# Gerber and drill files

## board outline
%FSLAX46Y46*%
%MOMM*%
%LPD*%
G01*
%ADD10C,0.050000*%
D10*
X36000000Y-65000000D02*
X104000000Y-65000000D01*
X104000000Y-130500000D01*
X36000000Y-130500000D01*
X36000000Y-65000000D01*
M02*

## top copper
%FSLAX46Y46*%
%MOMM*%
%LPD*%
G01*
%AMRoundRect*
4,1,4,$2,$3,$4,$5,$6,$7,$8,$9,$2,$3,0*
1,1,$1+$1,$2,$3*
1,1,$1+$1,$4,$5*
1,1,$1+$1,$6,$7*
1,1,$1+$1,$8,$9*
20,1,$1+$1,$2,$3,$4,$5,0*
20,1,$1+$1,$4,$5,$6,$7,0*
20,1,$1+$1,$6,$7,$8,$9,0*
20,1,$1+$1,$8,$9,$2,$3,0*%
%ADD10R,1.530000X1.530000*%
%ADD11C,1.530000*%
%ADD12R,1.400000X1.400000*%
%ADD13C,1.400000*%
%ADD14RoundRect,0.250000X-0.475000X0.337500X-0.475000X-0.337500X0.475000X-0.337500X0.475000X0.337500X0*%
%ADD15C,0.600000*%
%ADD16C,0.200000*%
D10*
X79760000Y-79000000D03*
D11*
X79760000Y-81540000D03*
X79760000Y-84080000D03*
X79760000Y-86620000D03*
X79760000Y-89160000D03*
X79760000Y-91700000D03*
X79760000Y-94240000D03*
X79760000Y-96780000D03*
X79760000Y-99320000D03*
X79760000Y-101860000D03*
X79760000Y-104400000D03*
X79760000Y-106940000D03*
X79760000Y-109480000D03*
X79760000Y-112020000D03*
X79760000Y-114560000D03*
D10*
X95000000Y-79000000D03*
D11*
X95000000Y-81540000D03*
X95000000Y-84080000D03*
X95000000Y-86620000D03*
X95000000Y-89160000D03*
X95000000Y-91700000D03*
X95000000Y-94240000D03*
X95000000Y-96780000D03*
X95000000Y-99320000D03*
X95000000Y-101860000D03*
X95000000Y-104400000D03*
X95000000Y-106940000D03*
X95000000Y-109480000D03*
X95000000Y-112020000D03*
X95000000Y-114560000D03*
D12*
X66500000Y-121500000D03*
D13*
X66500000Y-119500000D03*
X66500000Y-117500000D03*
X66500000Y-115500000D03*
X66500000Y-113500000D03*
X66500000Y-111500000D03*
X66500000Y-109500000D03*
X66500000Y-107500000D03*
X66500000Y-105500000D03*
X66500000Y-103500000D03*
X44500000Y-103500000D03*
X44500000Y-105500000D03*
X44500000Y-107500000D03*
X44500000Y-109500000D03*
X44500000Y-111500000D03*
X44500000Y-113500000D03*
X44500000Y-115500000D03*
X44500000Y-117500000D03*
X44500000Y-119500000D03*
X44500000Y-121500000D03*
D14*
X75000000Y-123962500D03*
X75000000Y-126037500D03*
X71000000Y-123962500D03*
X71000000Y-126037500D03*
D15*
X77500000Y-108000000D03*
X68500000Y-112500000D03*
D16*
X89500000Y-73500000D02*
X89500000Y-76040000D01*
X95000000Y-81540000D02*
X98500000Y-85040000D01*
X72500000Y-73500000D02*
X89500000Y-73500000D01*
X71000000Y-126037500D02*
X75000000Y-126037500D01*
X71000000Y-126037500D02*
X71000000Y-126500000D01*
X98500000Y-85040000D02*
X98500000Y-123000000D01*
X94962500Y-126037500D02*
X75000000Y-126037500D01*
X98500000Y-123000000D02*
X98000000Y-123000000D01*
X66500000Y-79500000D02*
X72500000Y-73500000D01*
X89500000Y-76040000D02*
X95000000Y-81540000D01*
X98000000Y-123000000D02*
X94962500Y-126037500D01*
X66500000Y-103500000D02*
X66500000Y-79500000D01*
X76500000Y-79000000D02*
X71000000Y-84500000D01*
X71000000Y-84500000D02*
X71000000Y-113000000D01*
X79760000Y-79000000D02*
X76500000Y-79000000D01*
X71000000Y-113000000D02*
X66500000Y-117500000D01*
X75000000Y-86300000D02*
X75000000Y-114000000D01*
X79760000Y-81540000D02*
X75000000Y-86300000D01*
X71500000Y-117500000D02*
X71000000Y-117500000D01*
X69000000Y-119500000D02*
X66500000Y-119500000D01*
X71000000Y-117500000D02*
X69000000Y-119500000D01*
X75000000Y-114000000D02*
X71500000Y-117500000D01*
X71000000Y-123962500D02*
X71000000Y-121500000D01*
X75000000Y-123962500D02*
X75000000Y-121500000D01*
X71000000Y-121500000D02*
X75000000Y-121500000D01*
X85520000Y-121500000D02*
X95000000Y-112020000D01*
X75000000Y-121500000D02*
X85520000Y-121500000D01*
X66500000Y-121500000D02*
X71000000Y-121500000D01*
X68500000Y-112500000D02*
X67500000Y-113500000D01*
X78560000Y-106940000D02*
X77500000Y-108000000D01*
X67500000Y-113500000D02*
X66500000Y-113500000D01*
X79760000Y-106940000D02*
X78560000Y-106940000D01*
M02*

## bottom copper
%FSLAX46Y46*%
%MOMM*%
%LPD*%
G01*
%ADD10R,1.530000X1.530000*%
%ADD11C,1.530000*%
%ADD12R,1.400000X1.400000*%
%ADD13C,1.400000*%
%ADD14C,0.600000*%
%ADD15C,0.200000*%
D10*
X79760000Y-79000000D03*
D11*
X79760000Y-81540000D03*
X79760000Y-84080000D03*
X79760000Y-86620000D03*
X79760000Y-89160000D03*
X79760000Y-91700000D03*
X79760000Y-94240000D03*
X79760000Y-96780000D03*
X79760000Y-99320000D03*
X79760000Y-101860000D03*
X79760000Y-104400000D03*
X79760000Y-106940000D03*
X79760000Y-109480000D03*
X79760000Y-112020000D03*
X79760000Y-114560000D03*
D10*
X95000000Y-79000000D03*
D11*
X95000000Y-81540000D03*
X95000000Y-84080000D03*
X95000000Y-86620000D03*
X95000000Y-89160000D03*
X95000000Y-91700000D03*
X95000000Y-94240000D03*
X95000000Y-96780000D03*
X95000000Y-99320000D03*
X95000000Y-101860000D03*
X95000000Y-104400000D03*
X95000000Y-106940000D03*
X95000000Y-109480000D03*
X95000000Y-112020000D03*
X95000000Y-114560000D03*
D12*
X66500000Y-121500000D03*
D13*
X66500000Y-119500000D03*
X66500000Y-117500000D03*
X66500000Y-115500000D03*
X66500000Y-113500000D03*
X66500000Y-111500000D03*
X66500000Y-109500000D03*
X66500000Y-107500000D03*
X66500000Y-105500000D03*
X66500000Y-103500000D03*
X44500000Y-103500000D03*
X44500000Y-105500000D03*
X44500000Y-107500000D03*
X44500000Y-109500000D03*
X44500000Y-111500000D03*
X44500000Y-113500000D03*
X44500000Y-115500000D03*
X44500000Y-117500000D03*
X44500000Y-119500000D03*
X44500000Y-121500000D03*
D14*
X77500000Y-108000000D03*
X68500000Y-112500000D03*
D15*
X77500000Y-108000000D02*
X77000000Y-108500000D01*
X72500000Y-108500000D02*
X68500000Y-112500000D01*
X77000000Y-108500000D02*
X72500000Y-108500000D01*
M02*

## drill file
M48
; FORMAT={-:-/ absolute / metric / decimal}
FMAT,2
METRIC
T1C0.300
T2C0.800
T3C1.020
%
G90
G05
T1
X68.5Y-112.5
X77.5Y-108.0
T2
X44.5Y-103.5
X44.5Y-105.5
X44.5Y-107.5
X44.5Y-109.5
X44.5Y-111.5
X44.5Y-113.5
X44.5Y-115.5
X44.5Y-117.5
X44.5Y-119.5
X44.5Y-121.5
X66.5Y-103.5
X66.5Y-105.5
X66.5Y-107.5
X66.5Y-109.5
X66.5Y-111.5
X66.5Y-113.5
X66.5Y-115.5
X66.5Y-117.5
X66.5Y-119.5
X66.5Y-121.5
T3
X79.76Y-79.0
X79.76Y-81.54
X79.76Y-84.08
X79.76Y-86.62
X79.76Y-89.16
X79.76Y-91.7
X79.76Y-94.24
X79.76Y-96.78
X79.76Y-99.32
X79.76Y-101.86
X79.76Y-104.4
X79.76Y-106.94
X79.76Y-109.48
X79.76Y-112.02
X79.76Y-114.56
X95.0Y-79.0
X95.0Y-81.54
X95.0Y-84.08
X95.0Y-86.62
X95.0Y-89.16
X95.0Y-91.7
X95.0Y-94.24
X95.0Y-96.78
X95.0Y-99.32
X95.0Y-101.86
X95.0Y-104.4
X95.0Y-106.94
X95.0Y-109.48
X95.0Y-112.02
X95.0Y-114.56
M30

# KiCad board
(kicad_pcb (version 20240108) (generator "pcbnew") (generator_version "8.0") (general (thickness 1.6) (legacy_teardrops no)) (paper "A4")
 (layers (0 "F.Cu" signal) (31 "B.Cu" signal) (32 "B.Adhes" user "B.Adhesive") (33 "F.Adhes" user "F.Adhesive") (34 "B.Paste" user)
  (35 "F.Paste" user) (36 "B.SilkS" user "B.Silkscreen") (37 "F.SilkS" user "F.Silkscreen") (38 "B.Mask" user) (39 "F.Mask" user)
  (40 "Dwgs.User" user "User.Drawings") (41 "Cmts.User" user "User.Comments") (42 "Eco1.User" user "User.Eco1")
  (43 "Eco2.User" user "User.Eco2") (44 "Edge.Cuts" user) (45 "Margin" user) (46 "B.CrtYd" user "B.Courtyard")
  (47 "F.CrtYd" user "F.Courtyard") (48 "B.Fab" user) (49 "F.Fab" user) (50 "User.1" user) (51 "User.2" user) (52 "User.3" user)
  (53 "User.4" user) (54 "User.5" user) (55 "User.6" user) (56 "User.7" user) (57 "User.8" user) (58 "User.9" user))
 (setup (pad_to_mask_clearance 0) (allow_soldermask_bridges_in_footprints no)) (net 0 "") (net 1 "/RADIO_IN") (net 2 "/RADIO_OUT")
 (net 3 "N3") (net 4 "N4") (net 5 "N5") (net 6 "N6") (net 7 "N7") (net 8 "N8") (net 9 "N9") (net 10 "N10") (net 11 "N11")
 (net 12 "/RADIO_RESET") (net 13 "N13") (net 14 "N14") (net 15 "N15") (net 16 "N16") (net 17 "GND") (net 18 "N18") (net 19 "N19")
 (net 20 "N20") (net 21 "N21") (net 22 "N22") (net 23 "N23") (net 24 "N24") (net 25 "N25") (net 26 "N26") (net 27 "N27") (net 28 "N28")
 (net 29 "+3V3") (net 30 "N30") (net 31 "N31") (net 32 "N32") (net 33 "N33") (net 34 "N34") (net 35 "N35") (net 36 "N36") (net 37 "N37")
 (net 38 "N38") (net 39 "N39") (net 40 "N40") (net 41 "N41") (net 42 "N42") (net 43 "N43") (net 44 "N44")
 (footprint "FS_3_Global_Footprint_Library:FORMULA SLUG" (layer "F.Cu") (at 41.44258 67.058544)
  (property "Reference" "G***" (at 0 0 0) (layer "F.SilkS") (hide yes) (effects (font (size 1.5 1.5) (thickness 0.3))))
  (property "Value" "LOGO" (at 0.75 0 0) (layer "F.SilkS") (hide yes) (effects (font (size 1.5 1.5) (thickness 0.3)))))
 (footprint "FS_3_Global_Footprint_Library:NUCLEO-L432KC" (layer "F.Cu") (at 87.38 95.215)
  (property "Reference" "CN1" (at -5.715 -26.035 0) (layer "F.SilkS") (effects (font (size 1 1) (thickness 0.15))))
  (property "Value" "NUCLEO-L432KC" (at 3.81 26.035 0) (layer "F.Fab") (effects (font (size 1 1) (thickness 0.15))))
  (pad "CN3_1" thru_hole rect (at -7.62 -16.215) (size 1.53 1.53) (drill 1.02) (layers "*.Cu" "*.Mask") (remove_unused_layers no)
   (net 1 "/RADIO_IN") (solder_mask_margin 0.102))
  (pad "CN3_2" thru_hole circle (at -7.62 -13.675) (size 1.53 1.53) (drill 1.02) (layers "*.Cu" "*.Mask") (remove_unused_layers no)
   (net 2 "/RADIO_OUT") (solder_mask_margin 0.102))
  (pad "CN3_3" thru_hole circle (at -7.62 -11.135) (size 1.53 1.53) (drill 1.02) (layers "*.Cu" "*.Mask") (remove_unused_layers no)
   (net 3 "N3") (solder_mask_margin 0.102))
  (pad "CN3_4" thru_hole circle (at -7.62 -8.595) (size 1.53 1.53) (drill 1.02) (layers "*.Cu" "*.Mask") (remove_unused_layers no)
   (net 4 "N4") (solder_mask_margin 0.102))
  (pad "CN3_5" thru_hole circle (at -7.62 -6.055) (size 1.53 1.53) (drill 1.02) (layers "*.Cu" "*.Mask") (remove_unused_layers no)
   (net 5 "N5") (solder_mask_margin 0.102))
  (pad "CN3_6" thru_hole circle (at -7.62 -3.515) (size 1.53 1.53) (drill 1.02) (layers "*.Cu" "*.Mask") (remove_unused_layers no)
   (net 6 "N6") (solder_mask_margin 0.102))
  (pad "CN3_7" thru_hole circle (at -7.62 -0.975) (size 1.53 1.53) (drill 1.02) (layers "*.Cu" "*.Mask") (remove_unused_layers no)
   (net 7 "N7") (solder_mask_margin 0.102))
  (pad "CN3_8" thru_hole circle (at -7.62 1.565) (size 1.53 1.53) (drill 1.02) (layers "*.Cu" "*.Mask") (remove_unused_layers no)
   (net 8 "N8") (solder_mask_margin 0.102))
  (pad "CN3_9" thru_hole circle (at -7.62 4.105) (size 1.53 1.53) (drill 1.02) (layers "*.Cu" "*.Mask") (remove_unused_layers no)
   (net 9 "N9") (solder_mask_margin 0.102))
  (pad "CN3_10" thru_hole circle (at -7.62 6.645) (size 1.53 1.53) (drill 1.02) (layers "*.Cu" "*.Mask") (remove_unused_layers no)
   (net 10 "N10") (solder_mask_margin 0.102))
  (pad "CN3_11" thru_hole circle (at -7.62 9.185) (size 1.53 1.53) (drill 1.02) (layers "*.Cu" "*.Mask") (remove_unused_layers no)
   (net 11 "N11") (solder_mask_margin 0.102))
  (pad "CN3_12" thru_hole circle (at -7.62 11.725) (size 1.53 1.53) (drill 1.02) (layers "*.Cu" "*.Mask") (remove_unused_layers no)
   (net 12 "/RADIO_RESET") (solder_mask_margin 0.102))
  (pad "CN3_13" thru_hole circle (at -7.62 14.265) (size 1.53 1.53) (drill 1.02) (layers "*.Cu" "*.Mask") (remove_unused_layers no)
   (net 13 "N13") (solder_mask_margin 0.102))
  (pad "CN3_14" thru_hole circle (at -7.62 16.805) (size 1.53 1.53) (drill 1.02) (layers "*.Cu" "*.Mask") (remove_unused_layers no)
   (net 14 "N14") (solder_mask_margin 0.102))
  (pad "CN3_15" thru_hole circle (at -7.62 19.345) (size 1.53 1.53) (drill 1.02) (layers "*.Cu" "*.Mask") (remove_unused_layers no)
   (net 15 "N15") (solder_mask_margin 0.102))
  (pad "CN4_1" thru_hole rect (at 7.62 -16.215) (size 1.53 1.53) (drill 1.02) (layers "*.Cu" "*.Mask") (remove_unused_layers no)
   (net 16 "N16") (solder_mask_margin 0.102))
  (pad "CN4_2" thru_hole circle (at 7.62 -13.675) (size 1.53 1.53) (drill 1.02) (layers "*.Cu" "*.Mask") (remove_unused_layers no)
   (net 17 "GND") (solder_mask_margin 0.102))
  (pad "CN4_3" thru_hole circle (at 7.62 -11.135) (size 1.53 1.53) (drill 1.02) (layers "*.Cu" "*.Mask") (remove_unused_layers no)
   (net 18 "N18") (solder_mask_margin 0.102))
  (pad "CN4_4" thru_hole circle (at 7.62 -8.595) (size 1.53 1.53) (drill 1.02) (layers "*.Cu" "*.Mask") (remove_unused_layers no)
   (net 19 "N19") (solder_mask_margin 0.102))
  (pad "CN4_5" thru_hole circle (at 7.62 -6.055) (size 1.53 1.53) (drill 1.02) (layers "*.Cu" "*.Mask") (remove_unused_layers no)
   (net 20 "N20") (solder_mask_margin 0.102))
  (pad "CN4_6" thru_hole circle (at 7.62 -3.515) (size 1.53 1.53) (drill 1.02) (layers "*.Cu" "*.Mask") (remove_unused_layers no)
   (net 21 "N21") (solder_mask_margin 0.102))
  (pad "CN4_7" thru_hole circle (at 7.62 -0.975) (size 1.53 1.53) (drill 1.02) (layers "*.Cu" "*.Mask") (remove_unused_layers no)
   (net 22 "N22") (solder_mask_margin 0.102))
  (pad "CN4_8" thru_hole circle (at 7.62 1.565) (size 1.53 1.53) (drill 1.02) (layers "*.Cu" "*.Mask") (remove_unused_layers no)
   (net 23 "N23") (solder_mask_margin 0.102))
  (pad "CN4_9" thru_hole circle (at 7.62 4.105) (size 1.53 1.53) (drill 1.02) (layers "*.Cu" "*.Mask") (remove_unused_layers no)
   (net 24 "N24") (solder_mask_margin 0.102))
  (pad "CN4_10" thru_hole circle (at 7.62 6.645) (size 1.53 1.53) (drill 1.02) (layers "*.Cu" "*.Mask") (remove_unused_layers no)
   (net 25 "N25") (solder_mask_margin 0.102))
  (pad "CN4_11" thru_hole circle (at 7.62 9.185) (size 1.53 1.53) (drill 1.02) (layers "*.Cu" "*.Mask") (remove_unused_layers no)
   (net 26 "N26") (solder_mask_margin 0.102))
  (pad "CN4_12" thru_hole circle (at 7.62 11.725) (size 1.53 1.53) (drill 1.02) (layers "*.Cu" "*.Mask") (remove_unused_layers no)
   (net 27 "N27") (solder_mask_margin 0.102))
  (pad "CN4_13" thru_hole circle (at 7.62 14.265) (size 1.53 1.53) (drill 1.02) (layers "*.Cu" "*.Mask") (remove_unused_layers no)
   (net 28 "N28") (solder_mask_margin 0.102))
  (pad "CN4_14" thru_hole circle (at 7.62 16.805) (size 1.53 1.53) (drill 1.02) (layers "*.Cu" "*.Mask") (remove_unused_layers no)
   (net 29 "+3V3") (solder_mask_margin 0.102))
  (pad "CN4_15" thru_hole circle (at 7.62 19.345) (size 1.53 1.53) (drill 1.02) (layers "*.Cu" "*.Mask") (remove_unused_layers no)
   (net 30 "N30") (solder_mask_margin 0.102)))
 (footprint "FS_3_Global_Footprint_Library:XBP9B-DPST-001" (layer "F.Cu") (at 55.5 112.75 180)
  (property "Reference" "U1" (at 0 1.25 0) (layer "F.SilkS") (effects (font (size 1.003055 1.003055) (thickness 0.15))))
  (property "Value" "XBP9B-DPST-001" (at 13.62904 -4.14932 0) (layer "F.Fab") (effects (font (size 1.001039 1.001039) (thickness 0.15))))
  (pad "1" thru_hole rect (at -11 -8.75 180) (size 1.4 1.4) (drill 0.8) (layers "*.Cu" "*.Mask") (remove_unused_layers no) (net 29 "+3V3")
   (solder_mask_margin 0.102))
  (pad "2" thru_hole circle (at -11 -6.75 180) (size 1.4 1.4) (drill 0.8) (layers "*.Cu" "*.Mask") (remove_unused_layers no)
   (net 2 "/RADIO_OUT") (solder_mask_margin 0.102))
  (pad "3" thru_hole circle (at -11 -4.75 180) (size 1.4 1.4) (drill 0.8) (layers "*.Cu" "*.Mask") (remove_unused_layers no)
   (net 1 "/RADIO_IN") (solder_mask_margin 0.102))
  (pad "4" thru_hole circle (at -11 -2.75 180) (size 1.4 1.4) (drill 0.8) (layers "*.Cu" "*.Mask") (remove_unused_layers no) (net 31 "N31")
   (solder_mask_margin 0.102))
  (pad "5" thru_hole circle (at -11 -0.75 180) (size 1.4 1.4) (drill 0.8) (layers "*.Cu" "*.Mask") (remove_unused_layers no)
   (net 12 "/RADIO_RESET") (solder_mask_margin 0.102))
  (pad "6" thru_hole circle (at -11 1.25 180) (size 1.4 1.4) (drill 0.8) (layers "*.Cu" "*.Mask") (remove_unused_layers no) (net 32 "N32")
   (solder_mask_margin 0.102))
  (pad "7" thru_hole circle (at -11 3.25 180) (size 1.4 1.4) (drill 0.8) (layers "*.Cu" "*.Mask") (remove_unused_layers no) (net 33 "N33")
   (solder_mask_margin 0.102))
  (pad "8" thru_hole circle (at -11 5.25 180) (size 1.4 1.4) (drill 0.8) (layers "*.Cu" "*.Mask") (remove_unused_layers no)
   (solder_mask_margin 0.102))
  (pad "9" thru_hole circle (at -11 7.25 180) (size 1.4 1.4) (drill 0.8) (layers "*.Cu" "*.Mask") (remove_unused_layers no) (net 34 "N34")
   (solder_mask_margin 0.102))
  (pad "10" thru_hole circle (at -11 9.25 180) (size 1.4 1.4) (drill 0.8) (layers "*.Cu" "*.Mask") (remove_unused_layers no) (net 17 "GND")
   (solder_mask_margin 0.102))
  (pad "11" thru_hole circle (at 11 9.25 180) (size 1.4 1.4) (drill 0.8) (layers "*.Cu" "*.Mask") (remove_unused_layers no) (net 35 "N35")
   (solder_mask_margin 0.102))
  (pad "12" thru_hole circle (at 11 7.25 180) (size 1.4 1.4) (drill 0.8) (layers "*.Cu" "*.Mask") (remove_unused_layers no) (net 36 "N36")
   (solder_mask_margin 0.102))
  (pad "13" thru_hole circle (at 11 5.25 180) (size 1.4 1.4) (drill 0.8) (layers "*.Cu" "*.Mask") (remove_unused_layers no) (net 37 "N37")
   (solder_mask_margin 0.102))
  (pad "14" thru_hole circle (at 11 3.25 180) (size 1.4 1.4) (drill 0.8) (layers "*.Cu" "*.Mask") (remove_unused_layers no) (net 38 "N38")
   (solder_mask_margin 0.102))
  (pad "15" thru_hole circle (at 11 1.25 180) (size 1.4 1.4) (drill 0.8) (layers "*.Cu" "*.Mask") (remove_unused_layers no) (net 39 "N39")
   (solder_mask_margin 0.102))
  (pad "16" thru_hole circle (at 11 -0.75 180) (size 1.4 1.4) (drill 0.8) (layers "*.Cu" "*.Mask") (remove_unused_layers no) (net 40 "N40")
   (solder_mask_margin 0.102))
  (pad "17" thru_hole circle (at 11 -2.75 180) (size 1.4 1.4) (drill 0.8) (layers "*.Cu" "*.Mask") (remove_unused_layers no) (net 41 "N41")
   (solder_mask_margin 0.102))
  (pad "18" thru_hole circle (at 11 -4.75 180) (size 1.4 1.4) (drill 0.8) (layers "*.Cu" "*.Mask") (remove_unused_layers no) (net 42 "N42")
   (solder_mask_margin 0.102))
  (pad "19" thru_hole circle (at 11 -6.75 180) (size 1.4 1.4) (drill 0.8) (layers "*.Cu" "*.Mask") (remove_unused_layers no) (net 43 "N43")
   (solder_mask_margin 0.102))
  (pad "20" thru_hole circle (at 11 -8.75 180) (size 1.4 1.4) (drill 0.8) (layers "*.Cu" "*.Mask") (remove_unused_layers no) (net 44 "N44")
   (solder_mask_margin 0.102)))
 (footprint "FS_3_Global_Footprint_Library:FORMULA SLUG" (layer "F.Cu") (at 105.44258 128.058544)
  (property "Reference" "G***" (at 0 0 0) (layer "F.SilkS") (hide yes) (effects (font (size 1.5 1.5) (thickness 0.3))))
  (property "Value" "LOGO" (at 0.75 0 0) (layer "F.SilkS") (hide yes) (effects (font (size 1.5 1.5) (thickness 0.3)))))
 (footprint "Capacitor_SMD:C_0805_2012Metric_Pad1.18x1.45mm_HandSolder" (layer "F.Cu") (at 75 125 -90)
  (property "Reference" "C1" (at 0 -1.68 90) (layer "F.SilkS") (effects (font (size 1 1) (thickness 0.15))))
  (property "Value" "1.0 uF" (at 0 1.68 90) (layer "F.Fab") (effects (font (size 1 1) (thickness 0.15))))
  (pad "1" smd roundrect (at -1.0375 0 270) (size 1.175 1.45) (layers "F.Cu" "F.Paste" "F.Mask") (roundrect_rratio 0.212766) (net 29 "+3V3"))
  (pad "2" smd roundrect (at 1.0375 0 270) (size 1.175 1.45) (layers "F.Cu" "F.Paste" "F.Mask") (roundrect_rratio 0.212766) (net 17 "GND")))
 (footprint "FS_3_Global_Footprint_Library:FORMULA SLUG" (layer "F.Cu") (at 104.94258 67.058544)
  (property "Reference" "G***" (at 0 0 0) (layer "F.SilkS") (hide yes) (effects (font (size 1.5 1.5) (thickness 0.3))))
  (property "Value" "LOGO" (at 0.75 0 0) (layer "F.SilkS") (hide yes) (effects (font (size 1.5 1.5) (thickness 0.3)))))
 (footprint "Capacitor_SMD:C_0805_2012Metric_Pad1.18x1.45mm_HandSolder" (layer "F.Cu") (at 71 125 -90)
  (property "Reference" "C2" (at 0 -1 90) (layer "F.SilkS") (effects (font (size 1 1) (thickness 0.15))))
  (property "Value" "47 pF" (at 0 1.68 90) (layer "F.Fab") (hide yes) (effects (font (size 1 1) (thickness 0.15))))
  (pad "1" smd roundrect (at -1.0375 0 270) (size 1.175 1.45) (layers "F.Cu" "F.Paste" "F.Mask") (roundrect_rratio 0.212766) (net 29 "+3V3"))
  (pad "2" smd roundrect (at 1.0375 0 270) (size 1.175 1.45) (layers "F.Cu" "F.Paste" "F.Mask") (roundrect_rratio 0.212766) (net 17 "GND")))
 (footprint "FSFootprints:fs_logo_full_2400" (layer "F.Cu") (at 49.5 83.5)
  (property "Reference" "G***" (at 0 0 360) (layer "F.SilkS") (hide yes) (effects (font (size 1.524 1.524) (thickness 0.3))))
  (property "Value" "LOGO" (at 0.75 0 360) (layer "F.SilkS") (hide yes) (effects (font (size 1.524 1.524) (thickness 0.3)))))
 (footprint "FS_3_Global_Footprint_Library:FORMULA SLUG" (layer "F.Cu") (at 40.94258 128.058544)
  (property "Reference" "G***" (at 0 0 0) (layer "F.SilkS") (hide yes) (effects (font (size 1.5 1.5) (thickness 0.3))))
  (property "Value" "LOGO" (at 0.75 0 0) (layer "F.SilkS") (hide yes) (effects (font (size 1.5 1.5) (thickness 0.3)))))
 (gr_rect (start 36 65) (end 104 130.5) (stroke (width 0.05) (type default)) (fill none) (layer "Edge.Cuts"))
 (segment (start 89.5 73.5) (end 89.5 76.04) (width 0.2) (layer "F.Cu") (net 17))
 (segment (start 95 81.54) (end 98.5 85.04) (width 0.2) (layer "F.Cu") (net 17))
 (segment (start 72.5 73.5) (end 89.5 73.5) (width 0.2) (layer "F.Cu") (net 17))
 (segment (start 71 126.0375) (end 75 126.0375) (width 0.2) (layer "F.Cu") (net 17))
 (segment (start 71 126.0375) (end 71 126.5) (width 0.2) (layer "F.Cu") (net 17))
 (segment (start 98.5 85.04) (end 98.5 123) (width 0.2) (layer "F.Cu") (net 17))
 (segment (start 94.9625 126.0375) (end 75 126.0375) (width 0.2) (layer "F.Cu") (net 17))
 (segment (start 98.5 123) (end 98 123) (width 0.2) (layer "F.Cu") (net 17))
 (segment (start 66.5 79.5) (end 72.5 73.5) (width 0.2) (layer "F.Cu") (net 17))
 (segment (start 89.5 76.04) (end 95 81.54) (width 0.2) (layer "F.Cu") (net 17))
 (segment (start 98 123) (end 94.9625 126.0375) (width 0.2) (layer "F.Cu") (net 17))
 (segment (start 66.5 103.5) (end 66.5 79.5) (width 0.2) (layer "F.Cu") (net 17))
 (segment (start 76.5 79) (end 71 84.5) (width 0.2) (layer "F.Cu") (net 1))
 (segment (start 71 84.5) (end 71 113) (width 0.2) (layer "F.Cu") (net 1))
 (segment (start 79.76 79) (end 76.5 79) (width 0.2) (layer "F.Cu") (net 1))
 (segment (start 71 113) (end 66.5 117.5) (width 0.2) (layer "F.Cu") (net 1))
 (segment (start 75 86.3) (end 75 114) (width 0.2) (layer "F.Cu") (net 2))
 (segment (start 79.76 81.54) (end 75 86.3) (width 0.2) (layer "F.Cu") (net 2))
 (segment (start 71.5 117.5) (end 71 117.5) (width 0.2) (layer "F.Cu") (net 2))
 (segment (start 69 119.5) (end 66.5 119.5) (width 0.2) (layer "F.Cu") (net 2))
 (segment (start 71 117.5) (end 69 119.5) (width 0.2) (layer "F.Cu") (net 2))
 (segment (start 75 114) (end 71.5 117.5) (width 0.2) (layer "F.Cu") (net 2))
 (segment (start 71 123.9625) (end 71 121.5) (width 0.2) (layer "F.Cu") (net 29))
 (segment (start 75 123.9625) (end 75 121.5) (width 0.2) (layer "F.Cu") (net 29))
 (segment (start 71 121.5) (end 75 121.5) (width 0.2) (layer "F.Cu") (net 29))
 (segment (start 85.52 121.5) (end 95 112.02) (width 0.2) (layer "F.Cu") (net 29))
 (segment (start 75 121.5) (end 85.52 121.5) (width 0.2) (layer "F.Cu") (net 29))
 (segment (start 66.5 121.5) (end 71 121.5) (width 0.2) (layer "F.Cu") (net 29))
 (segment (start 68.5 112.5) (end 67.5 113.5) (width 0.2) (layer "F.Cu") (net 12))
 (segment (start 78.56 106.94) (end 77.5 108) (width 0.2) (layer "F.Cu") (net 12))
 (segment (start 67.5 113.5) (end 66.5 113.5) (width 0.2) (layer "F.Cu") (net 12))
 (segment (start 79.76 106.94) (end 78.56 106.94) (width 0.2) (layer "F.Cu") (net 12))
 (via (at 77.5 108) (size 0.6) (drill 0.3) (layers "F.Cu" "B.Cu") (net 12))
 (via (at 68.5 112.5) (size 0.6) (drill 0.3) (layers "F.Cu" "B.Cu") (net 12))
 (segment (start 77.5 108) (end 77 108.5) (width 0.2) (layer "B.Cu") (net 12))
 (segment (start 72.5 108.5) (end 68.5 112.5) (width 0.2) (layer "B.Cu") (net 12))
 (segment (start 77 108.5) (end 72.5 108.5) (width 0.2) (layer "B.Cu") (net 12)))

